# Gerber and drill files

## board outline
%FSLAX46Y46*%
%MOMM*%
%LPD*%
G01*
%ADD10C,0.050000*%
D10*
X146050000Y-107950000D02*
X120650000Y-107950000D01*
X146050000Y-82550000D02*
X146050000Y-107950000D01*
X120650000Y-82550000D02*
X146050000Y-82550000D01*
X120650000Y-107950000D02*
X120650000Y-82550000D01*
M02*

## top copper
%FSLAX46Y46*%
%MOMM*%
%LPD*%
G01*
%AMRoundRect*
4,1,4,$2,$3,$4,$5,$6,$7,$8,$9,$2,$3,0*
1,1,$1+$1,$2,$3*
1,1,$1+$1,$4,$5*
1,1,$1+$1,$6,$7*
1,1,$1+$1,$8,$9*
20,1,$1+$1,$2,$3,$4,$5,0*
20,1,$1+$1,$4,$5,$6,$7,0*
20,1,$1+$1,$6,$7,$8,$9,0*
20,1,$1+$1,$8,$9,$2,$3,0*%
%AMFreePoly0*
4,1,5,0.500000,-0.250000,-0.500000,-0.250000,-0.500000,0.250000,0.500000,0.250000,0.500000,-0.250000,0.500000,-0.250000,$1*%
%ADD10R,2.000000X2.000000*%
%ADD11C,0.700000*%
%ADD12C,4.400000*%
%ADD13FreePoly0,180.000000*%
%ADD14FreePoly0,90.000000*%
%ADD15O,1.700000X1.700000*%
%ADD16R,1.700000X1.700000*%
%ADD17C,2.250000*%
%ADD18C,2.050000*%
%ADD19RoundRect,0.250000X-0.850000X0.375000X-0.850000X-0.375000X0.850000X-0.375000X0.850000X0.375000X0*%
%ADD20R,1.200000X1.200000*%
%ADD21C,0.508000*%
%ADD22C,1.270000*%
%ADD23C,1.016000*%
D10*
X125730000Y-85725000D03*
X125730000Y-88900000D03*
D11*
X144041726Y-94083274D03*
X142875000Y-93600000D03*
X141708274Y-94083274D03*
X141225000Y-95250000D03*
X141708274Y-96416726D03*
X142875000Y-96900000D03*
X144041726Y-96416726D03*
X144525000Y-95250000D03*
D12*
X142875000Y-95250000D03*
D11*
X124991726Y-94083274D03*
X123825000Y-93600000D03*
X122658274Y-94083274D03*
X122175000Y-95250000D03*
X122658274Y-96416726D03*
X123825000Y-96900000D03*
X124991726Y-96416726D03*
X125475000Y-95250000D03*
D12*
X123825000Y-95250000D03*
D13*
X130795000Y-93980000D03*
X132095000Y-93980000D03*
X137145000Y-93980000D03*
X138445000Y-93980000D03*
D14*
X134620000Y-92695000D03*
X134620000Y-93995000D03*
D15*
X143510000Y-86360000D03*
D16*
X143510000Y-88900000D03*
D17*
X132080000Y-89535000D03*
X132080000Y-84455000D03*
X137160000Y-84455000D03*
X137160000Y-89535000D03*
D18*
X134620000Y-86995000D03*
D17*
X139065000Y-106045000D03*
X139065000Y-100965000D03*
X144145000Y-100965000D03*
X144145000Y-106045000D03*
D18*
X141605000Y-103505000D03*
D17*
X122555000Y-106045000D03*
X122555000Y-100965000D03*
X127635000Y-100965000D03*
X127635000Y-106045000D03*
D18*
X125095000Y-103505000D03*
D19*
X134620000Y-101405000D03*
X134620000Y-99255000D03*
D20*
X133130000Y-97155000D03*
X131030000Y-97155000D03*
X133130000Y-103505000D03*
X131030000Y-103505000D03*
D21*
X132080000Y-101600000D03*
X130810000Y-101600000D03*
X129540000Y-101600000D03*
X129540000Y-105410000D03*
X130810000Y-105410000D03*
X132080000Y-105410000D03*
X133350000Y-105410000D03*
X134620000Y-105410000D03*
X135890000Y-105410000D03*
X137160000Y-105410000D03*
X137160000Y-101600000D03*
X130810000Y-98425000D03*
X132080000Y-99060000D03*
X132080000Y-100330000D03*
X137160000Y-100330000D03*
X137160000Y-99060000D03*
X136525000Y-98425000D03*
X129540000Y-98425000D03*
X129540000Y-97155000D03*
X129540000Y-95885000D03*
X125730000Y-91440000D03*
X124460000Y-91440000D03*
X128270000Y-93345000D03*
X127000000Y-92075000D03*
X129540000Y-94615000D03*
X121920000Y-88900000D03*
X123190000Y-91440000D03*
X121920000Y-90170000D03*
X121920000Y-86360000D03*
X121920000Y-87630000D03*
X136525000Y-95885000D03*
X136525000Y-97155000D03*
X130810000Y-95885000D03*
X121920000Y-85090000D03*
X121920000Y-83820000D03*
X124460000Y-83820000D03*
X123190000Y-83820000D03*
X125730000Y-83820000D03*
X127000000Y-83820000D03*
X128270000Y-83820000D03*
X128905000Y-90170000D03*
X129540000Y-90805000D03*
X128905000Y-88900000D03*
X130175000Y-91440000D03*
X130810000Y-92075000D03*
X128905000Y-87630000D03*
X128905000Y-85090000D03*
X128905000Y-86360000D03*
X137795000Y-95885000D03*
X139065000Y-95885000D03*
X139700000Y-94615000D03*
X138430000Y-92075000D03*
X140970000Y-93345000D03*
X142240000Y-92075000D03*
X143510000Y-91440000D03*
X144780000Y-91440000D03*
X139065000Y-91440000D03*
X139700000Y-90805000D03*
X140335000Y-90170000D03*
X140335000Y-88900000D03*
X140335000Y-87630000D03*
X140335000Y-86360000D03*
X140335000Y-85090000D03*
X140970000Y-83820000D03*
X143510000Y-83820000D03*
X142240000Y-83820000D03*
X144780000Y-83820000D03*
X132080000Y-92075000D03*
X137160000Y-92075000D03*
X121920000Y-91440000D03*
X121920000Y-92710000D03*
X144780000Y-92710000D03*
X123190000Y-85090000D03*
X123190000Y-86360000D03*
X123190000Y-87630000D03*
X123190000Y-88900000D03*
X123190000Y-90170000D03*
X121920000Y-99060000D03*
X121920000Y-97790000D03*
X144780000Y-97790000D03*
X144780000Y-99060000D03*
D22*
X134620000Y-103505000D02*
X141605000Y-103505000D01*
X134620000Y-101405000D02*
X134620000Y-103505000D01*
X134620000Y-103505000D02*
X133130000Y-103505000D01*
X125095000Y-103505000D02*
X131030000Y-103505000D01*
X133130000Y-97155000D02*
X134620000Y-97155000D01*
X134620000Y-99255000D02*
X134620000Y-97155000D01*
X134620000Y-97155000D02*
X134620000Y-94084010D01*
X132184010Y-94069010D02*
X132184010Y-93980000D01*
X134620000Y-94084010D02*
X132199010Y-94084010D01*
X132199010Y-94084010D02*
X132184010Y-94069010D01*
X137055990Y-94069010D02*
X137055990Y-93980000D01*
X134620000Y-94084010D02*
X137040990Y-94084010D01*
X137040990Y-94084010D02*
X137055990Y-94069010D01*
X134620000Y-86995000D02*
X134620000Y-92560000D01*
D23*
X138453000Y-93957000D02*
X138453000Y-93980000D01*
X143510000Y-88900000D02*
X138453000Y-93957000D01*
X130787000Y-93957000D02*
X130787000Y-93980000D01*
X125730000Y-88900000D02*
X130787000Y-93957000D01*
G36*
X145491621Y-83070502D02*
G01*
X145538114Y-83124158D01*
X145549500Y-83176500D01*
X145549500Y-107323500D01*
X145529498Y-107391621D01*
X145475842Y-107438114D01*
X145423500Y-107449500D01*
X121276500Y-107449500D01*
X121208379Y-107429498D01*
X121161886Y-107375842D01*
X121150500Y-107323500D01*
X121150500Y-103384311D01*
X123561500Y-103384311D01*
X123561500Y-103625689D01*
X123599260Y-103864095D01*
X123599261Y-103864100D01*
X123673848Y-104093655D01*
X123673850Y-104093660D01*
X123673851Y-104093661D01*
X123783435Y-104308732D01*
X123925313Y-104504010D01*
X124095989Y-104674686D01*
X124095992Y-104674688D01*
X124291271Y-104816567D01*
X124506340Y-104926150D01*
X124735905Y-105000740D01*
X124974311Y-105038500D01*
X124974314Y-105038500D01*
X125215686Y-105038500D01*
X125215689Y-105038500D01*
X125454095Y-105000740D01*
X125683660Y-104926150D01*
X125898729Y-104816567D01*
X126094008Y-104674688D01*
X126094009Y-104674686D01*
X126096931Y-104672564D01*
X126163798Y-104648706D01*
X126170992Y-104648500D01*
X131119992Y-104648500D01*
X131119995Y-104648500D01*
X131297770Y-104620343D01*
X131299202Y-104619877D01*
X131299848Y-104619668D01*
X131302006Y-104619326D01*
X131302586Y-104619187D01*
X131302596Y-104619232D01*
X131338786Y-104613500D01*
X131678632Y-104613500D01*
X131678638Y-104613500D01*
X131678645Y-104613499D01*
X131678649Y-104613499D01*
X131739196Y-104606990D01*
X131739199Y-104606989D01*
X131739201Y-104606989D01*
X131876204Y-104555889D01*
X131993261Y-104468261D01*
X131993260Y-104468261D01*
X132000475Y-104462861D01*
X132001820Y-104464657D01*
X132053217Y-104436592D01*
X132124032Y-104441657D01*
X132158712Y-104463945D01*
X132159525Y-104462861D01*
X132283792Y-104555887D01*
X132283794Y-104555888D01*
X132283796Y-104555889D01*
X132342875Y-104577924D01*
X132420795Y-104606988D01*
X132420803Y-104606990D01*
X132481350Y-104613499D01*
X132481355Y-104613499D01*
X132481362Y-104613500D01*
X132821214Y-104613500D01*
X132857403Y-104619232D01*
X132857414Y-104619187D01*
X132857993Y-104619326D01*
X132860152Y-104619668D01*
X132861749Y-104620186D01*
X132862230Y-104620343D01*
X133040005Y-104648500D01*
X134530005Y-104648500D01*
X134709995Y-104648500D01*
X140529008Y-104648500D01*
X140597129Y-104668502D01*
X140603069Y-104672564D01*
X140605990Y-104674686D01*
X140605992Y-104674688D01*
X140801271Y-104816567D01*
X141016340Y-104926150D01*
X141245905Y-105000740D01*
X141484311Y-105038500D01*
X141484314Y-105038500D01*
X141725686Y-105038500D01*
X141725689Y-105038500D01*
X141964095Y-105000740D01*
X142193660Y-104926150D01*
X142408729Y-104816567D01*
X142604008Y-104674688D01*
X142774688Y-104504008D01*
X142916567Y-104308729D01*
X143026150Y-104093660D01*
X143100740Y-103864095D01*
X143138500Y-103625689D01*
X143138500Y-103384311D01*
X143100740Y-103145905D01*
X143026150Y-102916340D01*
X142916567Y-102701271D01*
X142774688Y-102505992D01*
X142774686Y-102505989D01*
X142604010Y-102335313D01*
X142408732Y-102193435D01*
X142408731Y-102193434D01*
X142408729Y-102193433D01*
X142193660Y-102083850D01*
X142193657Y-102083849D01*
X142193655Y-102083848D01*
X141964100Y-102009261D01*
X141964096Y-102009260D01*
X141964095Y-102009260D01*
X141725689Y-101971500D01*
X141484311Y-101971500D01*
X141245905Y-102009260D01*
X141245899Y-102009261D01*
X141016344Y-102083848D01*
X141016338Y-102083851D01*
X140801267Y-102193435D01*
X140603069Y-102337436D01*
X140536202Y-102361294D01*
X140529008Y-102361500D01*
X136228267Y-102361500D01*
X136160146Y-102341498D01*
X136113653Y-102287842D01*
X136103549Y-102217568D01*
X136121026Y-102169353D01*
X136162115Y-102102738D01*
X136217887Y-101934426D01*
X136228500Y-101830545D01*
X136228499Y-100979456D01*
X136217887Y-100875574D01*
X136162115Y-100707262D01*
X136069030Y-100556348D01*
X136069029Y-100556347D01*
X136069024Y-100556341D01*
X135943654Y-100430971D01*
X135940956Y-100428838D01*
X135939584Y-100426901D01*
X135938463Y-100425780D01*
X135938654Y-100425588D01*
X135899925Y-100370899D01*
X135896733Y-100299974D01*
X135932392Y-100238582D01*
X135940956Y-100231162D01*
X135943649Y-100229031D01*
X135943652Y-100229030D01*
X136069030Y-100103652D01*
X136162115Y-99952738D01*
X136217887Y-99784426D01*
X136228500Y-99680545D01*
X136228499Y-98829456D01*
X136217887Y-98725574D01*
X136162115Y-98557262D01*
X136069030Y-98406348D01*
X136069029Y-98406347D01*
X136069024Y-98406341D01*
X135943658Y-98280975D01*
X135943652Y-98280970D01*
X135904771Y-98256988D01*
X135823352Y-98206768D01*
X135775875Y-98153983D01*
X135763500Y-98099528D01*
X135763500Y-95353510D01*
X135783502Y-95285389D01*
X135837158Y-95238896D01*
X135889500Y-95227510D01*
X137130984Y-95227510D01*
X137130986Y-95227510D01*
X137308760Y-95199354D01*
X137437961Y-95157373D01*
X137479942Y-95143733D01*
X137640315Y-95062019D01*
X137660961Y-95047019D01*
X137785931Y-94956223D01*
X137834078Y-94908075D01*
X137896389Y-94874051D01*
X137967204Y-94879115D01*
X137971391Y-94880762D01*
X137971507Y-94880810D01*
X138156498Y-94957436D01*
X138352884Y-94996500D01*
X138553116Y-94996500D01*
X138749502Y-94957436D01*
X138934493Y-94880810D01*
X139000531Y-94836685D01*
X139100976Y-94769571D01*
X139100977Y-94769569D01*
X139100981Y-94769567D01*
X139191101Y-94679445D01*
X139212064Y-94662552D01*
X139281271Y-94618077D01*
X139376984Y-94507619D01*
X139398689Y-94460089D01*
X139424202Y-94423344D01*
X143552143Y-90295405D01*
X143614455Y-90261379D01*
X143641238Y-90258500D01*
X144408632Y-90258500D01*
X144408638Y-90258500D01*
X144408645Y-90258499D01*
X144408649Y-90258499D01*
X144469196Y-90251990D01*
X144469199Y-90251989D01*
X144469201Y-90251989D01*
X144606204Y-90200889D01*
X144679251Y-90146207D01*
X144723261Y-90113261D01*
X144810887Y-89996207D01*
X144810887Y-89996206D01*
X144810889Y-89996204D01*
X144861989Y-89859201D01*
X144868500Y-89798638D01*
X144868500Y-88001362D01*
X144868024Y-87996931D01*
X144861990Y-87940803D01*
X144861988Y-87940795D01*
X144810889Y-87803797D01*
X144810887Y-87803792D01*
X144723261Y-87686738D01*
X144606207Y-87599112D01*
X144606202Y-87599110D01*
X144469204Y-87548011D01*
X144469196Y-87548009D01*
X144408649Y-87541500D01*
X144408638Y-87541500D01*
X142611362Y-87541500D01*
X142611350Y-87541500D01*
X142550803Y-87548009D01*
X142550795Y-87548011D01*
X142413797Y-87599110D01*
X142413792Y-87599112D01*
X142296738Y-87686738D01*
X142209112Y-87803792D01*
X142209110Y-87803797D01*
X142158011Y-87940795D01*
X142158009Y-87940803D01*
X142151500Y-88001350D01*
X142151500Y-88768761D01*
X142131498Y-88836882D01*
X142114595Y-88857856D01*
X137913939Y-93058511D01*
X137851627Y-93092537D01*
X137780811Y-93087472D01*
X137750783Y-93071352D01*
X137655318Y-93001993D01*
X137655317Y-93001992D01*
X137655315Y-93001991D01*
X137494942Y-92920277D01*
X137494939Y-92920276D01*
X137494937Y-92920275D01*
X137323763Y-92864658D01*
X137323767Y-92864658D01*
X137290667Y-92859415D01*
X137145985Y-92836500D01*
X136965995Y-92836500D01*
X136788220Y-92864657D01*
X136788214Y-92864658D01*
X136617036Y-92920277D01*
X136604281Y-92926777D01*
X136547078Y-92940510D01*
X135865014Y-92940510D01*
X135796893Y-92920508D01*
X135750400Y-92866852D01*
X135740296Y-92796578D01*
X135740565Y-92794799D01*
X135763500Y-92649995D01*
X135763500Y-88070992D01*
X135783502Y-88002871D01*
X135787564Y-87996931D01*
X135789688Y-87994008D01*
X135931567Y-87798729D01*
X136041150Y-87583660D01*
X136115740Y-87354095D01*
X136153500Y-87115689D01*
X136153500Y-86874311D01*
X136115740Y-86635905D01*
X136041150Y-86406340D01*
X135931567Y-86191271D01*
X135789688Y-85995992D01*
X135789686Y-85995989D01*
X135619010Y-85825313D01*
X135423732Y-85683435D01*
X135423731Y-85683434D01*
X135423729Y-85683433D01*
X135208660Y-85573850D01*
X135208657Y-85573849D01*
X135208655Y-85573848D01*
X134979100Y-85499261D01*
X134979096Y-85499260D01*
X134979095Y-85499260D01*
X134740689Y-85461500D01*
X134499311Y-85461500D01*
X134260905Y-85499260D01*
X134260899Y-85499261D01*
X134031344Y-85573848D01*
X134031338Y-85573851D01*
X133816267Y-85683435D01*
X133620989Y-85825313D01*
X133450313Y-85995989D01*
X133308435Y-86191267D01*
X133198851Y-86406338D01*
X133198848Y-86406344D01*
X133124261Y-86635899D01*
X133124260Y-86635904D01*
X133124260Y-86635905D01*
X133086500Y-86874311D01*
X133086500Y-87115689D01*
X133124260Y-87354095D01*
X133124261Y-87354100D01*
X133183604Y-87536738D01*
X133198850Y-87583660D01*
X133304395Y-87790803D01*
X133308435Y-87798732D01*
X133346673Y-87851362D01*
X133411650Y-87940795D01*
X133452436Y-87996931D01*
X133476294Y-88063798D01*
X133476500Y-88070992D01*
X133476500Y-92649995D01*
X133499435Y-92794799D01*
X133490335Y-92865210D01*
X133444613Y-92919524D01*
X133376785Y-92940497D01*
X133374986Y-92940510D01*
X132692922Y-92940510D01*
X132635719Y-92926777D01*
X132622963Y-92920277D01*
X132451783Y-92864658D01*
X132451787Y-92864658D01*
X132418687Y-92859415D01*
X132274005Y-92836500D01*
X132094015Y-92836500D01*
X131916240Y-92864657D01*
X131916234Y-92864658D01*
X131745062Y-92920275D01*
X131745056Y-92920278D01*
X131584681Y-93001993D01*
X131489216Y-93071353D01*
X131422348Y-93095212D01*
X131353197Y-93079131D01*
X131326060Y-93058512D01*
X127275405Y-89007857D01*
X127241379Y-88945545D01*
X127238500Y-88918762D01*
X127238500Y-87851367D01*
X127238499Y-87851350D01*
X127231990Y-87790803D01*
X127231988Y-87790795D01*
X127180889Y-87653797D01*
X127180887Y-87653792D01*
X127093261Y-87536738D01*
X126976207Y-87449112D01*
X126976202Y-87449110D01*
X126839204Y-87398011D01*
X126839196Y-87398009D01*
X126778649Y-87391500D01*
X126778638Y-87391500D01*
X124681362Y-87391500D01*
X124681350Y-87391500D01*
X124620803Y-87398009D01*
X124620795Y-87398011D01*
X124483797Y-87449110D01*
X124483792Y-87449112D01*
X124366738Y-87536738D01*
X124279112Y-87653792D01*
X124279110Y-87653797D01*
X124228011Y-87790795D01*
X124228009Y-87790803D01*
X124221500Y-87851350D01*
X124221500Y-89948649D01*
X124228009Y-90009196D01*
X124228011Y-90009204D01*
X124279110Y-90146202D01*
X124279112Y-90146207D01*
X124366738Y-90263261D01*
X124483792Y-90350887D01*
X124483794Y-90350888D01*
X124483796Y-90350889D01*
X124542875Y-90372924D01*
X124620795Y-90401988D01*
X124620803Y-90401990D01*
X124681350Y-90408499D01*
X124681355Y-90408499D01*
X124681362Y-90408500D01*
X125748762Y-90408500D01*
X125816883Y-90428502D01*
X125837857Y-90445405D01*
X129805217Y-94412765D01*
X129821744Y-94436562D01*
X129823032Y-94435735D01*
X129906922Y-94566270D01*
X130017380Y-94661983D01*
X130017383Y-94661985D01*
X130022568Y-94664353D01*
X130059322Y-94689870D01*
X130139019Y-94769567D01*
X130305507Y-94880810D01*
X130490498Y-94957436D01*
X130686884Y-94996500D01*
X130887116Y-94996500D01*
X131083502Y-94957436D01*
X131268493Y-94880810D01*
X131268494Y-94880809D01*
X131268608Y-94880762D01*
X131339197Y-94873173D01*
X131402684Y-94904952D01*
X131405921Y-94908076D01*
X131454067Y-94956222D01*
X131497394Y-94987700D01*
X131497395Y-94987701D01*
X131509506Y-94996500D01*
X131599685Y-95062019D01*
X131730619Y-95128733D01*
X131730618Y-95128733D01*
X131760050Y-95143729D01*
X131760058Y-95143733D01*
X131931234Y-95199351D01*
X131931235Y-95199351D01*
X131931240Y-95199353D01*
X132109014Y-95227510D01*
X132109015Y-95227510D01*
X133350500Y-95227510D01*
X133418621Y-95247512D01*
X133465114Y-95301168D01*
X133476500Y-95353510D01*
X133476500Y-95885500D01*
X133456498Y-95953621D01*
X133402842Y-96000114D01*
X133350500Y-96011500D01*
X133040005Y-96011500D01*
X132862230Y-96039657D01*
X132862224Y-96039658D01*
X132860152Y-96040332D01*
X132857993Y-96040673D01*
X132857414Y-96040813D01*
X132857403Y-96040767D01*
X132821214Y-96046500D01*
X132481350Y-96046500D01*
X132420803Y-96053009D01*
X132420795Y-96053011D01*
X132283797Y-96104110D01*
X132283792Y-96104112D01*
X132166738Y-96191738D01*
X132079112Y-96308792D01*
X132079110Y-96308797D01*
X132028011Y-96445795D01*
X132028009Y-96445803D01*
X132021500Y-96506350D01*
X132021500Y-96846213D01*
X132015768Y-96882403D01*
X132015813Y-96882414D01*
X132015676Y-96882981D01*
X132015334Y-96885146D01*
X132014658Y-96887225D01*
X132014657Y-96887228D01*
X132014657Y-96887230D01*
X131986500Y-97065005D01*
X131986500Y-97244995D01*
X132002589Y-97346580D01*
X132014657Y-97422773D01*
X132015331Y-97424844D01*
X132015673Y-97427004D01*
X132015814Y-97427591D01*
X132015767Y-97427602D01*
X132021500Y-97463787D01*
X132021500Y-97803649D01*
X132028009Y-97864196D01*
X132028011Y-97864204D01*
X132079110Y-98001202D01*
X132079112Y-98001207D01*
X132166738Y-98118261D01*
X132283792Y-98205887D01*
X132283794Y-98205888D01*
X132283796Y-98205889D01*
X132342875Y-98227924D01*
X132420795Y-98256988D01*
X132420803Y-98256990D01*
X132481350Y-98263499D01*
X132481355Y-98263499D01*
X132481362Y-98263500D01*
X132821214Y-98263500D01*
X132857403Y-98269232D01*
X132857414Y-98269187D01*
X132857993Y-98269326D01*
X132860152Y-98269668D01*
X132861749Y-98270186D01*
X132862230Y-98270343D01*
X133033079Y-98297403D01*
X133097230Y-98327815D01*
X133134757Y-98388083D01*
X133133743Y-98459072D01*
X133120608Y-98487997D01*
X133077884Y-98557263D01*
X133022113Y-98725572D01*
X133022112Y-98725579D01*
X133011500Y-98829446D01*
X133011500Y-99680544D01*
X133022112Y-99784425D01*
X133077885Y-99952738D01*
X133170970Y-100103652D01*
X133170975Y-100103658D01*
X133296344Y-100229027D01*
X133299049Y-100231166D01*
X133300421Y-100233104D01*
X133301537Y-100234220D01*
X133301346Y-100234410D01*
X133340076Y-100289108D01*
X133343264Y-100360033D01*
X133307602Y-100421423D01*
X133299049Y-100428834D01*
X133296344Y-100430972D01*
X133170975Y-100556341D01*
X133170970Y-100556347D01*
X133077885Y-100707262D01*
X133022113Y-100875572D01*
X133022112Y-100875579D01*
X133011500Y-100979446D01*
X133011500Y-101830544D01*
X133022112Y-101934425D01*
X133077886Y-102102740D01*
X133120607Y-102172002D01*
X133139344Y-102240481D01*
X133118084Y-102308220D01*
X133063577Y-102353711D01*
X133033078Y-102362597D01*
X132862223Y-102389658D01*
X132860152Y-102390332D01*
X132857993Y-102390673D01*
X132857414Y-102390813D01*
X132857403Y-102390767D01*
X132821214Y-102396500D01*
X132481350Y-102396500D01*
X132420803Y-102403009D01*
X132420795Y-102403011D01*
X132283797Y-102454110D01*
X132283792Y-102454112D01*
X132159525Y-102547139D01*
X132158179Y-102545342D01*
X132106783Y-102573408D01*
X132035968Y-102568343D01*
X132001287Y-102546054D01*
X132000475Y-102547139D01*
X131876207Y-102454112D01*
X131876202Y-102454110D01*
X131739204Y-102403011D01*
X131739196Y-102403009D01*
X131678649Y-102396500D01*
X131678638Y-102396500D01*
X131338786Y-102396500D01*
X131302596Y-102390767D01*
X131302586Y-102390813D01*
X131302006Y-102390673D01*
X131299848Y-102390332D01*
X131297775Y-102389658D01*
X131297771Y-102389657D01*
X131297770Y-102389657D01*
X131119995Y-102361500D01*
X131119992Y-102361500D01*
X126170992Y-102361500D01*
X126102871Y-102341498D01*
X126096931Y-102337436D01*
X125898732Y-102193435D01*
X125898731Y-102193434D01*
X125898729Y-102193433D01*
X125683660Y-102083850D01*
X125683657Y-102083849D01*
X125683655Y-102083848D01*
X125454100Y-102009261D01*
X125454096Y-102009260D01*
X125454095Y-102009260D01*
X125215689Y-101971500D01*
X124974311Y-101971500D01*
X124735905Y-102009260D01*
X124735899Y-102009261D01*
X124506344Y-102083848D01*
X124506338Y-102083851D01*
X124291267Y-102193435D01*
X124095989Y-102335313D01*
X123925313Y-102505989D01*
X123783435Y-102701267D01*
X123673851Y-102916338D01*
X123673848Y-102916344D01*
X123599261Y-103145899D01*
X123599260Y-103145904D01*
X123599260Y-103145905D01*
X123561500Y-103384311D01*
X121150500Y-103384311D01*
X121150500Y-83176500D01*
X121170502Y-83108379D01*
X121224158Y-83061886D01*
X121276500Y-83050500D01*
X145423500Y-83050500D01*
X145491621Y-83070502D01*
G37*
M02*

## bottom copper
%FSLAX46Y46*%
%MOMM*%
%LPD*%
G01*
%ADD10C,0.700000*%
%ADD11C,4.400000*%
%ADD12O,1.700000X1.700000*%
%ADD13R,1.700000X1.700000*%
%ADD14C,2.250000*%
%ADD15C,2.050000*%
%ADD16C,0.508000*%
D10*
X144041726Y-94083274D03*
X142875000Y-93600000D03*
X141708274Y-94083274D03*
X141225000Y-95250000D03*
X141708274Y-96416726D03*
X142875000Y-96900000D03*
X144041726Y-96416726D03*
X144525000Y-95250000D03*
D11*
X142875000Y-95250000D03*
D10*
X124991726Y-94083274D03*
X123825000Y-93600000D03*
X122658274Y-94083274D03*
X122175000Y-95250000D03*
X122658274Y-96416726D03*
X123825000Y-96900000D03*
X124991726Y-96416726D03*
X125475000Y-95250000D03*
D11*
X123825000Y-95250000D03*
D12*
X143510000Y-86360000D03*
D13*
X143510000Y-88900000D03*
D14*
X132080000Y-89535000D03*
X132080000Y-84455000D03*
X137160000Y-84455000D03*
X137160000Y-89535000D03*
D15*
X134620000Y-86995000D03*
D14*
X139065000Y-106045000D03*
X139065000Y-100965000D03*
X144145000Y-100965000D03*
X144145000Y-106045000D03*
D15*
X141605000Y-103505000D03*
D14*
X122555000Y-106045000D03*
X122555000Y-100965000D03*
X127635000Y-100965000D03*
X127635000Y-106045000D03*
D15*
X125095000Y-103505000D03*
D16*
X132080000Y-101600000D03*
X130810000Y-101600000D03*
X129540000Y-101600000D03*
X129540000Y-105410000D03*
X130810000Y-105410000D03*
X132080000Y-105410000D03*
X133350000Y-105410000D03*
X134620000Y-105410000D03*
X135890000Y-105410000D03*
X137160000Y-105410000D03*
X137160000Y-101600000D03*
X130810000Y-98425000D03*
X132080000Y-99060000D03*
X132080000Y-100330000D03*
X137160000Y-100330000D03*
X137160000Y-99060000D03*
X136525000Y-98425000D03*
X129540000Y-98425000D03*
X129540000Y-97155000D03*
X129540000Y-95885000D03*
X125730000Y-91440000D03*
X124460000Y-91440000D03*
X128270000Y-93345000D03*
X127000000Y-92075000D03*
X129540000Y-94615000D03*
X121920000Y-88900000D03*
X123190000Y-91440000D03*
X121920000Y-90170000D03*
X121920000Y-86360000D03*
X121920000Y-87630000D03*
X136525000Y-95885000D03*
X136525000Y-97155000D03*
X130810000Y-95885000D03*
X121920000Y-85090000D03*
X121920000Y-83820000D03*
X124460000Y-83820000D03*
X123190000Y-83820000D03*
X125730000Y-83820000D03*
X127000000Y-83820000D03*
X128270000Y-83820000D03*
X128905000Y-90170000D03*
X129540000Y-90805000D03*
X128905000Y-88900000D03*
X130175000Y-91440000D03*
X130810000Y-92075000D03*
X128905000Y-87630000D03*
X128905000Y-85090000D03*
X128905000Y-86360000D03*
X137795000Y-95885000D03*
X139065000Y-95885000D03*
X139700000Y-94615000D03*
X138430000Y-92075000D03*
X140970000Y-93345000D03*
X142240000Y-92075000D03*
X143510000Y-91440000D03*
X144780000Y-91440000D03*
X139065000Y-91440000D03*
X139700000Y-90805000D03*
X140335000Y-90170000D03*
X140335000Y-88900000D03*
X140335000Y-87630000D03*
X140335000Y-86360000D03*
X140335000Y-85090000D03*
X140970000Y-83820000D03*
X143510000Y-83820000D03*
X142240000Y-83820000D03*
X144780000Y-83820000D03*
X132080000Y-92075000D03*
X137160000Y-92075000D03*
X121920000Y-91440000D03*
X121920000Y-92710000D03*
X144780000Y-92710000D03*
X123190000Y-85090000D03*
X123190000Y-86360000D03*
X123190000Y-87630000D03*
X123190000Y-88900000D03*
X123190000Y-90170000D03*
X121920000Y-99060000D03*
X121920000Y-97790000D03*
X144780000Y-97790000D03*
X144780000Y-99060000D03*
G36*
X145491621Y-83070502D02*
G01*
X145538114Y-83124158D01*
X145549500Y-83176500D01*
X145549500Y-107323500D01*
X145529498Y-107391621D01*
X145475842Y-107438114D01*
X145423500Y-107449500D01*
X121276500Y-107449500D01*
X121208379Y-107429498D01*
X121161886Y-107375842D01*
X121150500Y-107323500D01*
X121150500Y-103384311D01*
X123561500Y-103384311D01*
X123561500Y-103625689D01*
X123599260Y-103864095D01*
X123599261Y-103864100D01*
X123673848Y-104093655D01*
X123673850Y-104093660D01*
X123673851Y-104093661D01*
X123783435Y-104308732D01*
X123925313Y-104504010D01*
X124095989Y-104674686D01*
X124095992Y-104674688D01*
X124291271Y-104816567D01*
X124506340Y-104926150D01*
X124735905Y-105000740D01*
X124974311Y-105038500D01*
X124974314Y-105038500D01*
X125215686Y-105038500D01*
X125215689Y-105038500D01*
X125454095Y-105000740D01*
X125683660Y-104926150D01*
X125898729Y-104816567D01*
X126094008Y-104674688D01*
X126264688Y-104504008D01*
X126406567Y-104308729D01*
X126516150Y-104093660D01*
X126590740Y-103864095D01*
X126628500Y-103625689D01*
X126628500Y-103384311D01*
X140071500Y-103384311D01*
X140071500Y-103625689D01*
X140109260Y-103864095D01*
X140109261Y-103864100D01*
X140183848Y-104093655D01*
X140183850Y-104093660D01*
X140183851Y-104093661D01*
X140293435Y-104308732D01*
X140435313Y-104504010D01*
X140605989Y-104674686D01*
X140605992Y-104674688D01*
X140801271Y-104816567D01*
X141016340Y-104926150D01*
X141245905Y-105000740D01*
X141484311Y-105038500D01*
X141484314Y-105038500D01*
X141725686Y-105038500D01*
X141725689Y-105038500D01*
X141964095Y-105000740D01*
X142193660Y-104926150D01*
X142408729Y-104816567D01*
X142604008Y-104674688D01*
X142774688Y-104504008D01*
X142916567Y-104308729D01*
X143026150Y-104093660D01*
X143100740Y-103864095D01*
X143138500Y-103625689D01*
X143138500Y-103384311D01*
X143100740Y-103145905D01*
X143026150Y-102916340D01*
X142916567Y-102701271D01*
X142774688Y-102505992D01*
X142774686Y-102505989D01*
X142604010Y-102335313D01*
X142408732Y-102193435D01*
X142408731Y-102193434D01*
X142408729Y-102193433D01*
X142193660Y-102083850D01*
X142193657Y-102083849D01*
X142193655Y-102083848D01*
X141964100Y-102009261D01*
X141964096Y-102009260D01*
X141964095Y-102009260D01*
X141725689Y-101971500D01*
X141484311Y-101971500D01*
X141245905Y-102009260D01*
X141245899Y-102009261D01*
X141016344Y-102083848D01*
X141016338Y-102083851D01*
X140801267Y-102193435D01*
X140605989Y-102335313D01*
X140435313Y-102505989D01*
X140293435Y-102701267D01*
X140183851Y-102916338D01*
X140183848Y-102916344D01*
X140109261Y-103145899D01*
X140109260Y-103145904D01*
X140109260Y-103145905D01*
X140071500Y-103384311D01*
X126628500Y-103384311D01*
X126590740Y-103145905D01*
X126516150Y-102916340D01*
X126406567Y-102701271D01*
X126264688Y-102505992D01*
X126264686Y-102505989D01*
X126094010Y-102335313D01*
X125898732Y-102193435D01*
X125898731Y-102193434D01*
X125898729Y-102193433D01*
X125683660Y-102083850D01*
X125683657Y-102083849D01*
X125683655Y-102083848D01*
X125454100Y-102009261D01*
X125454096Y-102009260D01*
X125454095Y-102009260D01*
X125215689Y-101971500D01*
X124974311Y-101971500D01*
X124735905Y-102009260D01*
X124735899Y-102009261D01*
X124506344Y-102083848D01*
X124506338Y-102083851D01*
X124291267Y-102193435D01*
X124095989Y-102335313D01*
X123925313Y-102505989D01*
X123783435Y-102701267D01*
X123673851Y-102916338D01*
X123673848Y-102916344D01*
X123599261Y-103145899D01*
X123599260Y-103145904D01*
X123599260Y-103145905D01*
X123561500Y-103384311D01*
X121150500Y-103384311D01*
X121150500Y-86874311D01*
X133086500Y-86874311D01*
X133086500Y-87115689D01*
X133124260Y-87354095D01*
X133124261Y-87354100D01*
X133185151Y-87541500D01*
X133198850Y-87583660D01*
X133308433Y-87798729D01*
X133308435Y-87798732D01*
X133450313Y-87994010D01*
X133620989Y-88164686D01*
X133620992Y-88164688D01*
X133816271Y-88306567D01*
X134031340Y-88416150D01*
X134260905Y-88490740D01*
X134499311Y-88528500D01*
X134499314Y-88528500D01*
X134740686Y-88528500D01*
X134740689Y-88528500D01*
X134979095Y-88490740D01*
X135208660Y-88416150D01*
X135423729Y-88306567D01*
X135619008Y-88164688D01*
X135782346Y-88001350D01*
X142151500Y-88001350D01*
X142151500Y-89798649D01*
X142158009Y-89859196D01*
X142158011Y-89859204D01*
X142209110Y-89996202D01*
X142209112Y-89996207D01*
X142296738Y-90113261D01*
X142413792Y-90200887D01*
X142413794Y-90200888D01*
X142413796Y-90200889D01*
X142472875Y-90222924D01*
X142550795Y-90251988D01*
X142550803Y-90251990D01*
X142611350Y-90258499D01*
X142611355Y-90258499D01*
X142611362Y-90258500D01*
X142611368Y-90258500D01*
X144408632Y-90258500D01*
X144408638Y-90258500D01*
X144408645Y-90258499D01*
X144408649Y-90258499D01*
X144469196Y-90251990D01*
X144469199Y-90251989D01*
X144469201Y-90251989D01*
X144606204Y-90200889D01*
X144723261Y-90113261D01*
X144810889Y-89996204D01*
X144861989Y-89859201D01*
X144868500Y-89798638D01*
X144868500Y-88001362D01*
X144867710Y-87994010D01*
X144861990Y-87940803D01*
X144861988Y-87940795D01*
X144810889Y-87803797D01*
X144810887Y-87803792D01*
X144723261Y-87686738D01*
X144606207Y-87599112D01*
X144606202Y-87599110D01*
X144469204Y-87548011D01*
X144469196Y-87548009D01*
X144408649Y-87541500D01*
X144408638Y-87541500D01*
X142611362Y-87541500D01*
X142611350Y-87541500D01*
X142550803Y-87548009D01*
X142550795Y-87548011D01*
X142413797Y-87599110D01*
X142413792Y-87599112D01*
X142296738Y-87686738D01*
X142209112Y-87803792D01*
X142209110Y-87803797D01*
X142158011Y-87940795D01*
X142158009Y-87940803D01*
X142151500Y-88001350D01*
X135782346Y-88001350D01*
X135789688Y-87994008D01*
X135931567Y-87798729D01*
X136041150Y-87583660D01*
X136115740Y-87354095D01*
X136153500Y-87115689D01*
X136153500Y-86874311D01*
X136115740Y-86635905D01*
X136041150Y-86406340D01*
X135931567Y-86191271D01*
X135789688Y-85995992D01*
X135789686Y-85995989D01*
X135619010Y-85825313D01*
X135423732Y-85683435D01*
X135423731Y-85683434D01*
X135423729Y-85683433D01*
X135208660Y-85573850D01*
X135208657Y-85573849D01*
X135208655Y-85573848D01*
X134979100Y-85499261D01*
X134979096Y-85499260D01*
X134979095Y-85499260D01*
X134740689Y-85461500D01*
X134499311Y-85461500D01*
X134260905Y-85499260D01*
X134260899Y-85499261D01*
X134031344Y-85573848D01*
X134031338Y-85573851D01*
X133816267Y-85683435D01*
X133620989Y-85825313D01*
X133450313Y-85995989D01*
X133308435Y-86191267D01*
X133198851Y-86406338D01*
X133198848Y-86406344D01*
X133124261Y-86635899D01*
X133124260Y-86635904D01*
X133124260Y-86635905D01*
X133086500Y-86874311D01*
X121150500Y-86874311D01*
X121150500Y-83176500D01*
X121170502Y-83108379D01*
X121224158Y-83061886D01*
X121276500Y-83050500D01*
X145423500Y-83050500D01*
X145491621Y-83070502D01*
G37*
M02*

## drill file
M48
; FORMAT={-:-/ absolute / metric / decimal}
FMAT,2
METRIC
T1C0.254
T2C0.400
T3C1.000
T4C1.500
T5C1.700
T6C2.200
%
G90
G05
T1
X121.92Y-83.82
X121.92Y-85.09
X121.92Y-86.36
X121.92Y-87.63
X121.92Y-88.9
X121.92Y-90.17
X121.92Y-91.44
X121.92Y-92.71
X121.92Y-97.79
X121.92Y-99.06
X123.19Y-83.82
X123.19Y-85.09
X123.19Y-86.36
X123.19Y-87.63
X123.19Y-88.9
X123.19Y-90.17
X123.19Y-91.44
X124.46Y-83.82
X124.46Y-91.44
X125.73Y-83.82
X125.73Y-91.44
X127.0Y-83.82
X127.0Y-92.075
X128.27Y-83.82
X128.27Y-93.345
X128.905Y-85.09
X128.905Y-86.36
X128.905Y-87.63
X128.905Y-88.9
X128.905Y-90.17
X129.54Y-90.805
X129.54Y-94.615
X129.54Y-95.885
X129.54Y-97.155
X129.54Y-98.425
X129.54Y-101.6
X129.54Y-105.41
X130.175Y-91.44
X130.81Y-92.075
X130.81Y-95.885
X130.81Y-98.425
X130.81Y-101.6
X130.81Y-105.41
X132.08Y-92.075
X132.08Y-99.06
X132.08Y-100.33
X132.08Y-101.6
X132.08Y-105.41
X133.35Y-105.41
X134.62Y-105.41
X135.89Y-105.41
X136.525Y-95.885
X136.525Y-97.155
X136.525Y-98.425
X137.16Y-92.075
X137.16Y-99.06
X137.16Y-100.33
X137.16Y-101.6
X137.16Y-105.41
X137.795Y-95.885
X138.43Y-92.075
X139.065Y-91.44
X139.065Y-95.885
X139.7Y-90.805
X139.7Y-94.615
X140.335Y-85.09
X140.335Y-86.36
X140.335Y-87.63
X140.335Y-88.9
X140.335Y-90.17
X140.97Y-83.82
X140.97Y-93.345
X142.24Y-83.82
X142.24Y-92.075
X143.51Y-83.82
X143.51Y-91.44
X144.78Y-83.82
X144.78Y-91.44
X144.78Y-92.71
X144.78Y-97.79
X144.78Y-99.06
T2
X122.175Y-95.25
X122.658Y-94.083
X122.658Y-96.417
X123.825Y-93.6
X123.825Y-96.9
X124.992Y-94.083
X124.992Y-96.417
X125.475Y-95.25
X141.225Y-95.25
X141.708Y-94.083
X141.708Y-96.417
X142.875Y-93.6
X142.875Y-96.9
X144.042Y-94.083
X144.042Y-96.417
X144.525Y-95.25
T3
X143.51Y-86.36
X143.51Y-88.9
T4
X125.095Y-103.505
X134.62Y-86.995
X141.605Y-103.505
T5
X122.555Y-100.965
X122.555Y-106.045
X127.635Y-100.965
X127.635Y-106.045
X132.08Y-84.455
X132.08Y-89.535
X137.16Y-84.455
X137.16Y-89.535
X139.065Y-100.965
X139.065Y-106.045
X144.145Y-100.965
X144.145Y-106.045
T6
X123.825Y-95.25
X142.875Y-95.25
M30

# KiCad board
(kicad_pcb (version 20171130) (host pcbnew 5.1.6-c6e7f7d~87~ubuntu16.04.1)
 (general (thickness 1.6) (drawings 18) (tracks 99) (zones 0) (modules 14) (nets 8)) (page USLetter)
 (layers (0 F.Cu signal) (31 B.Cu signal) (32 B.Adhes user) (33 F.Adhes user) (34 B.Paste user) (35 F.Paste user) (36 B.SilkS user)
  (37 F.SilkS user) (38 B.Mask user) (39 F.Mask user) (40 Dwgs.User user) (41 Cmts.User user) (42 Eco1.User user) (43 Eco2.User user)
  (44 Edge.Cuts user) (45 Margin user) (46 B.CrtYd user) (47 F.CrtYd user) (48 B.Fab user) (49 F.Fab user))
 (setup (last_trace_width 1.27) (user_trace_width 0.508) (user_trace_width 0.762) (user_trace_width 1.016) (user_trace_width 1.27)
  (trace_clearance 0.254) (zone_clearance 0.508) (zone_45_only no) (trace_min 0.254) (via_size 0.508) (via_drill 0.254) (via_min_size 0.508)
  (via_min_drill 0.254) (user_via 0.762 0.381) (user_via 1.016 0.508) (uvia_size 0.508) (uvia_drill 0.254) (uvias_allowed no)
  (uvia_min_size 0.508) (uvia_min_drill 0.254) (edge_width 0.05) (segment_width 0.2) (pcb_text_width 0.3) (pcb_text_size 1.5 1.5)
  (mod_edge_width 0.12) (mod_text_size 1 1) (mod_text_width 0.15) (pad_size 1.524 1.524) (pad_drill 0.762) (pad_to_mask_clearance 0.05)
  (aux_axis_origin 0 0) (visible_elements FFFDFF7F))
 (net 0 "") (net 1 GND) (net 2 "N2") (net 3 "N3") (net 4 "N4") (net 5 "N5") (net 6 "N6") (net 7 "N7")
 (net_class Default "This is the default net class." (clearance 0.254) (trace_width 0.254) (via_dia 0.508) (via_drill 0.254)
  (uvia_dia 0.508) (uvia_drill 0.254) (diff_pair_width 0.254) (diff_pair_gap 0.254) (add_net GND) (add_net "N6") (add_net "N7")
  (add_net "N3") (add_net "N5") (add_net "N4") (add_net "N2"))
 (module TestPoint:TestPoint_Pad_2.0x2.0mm (layer F.Cu) (at 125.73 85.725)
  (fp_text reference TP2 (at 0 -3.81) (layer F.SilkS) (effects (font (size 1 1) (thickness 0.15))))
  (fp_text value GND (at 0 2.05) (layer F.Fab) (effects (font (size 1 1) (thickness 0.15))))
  (pad 1 smd rect (at 0 0) (size 2 2) (layers F.Cu F.Mask) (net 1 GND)))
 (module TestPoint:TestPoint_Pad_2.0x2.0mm (layer F.Cu) (at 125.73 88.9)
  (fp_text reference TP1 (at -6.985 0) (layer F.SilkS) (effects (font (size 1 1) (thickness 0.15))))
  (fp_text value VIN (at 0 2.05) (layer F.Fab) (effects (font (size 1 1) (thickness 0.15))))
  (pad 1 smd rect (at 0 0) (size 2 2) (layers F.Cu F.Mask) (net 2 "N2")))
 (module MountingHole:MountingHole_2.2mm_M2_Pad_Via (layer F.Cu) (at 142.875 95.25)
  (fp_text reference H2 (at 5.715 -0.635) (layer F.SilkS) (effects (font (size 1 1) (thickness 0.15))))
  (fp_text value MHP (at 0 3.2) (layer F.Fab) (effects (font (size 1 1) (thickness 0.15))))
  (pad 1 thru_hole circle (at 1.166726 -1.166726) (size 0.7 0.7) (drill 0.4) (layers *.Cu *.Mask) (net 1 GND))
  (pad 1 thru_hole circle (at 0 -1.65) (size 0.7 0.7) (drill 0.4) (layers *.Cu *.Mask) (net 1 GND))
  (pad 1 thru_hole circle (at -1.166726 -1.166726) (size 0.7 0.7) (drill 0.4) (layers *.Cu *.Mask) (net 1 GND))
  (pad 1 thru_hole circle (at -1.65 0) (size 0.7 0.7) (drill 0.4) (layers *.Cu *.Mask) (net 1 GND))
  (pad 1 thru_hole circle (at -1.166726 1.166726) (size 0.7 0.7) (drill 0.4) (layers *.Cu *.Mask) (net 1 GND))
  (pad 1 thru_hole circle (at 0 1.65) (size 0.7 0.7) (drill 0.4) (layers *.Cu *.Mask) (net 1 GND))
  (pad 1 thru_hole circle (at 1.166726 1.166726) (size 0.7 0.7) (drill 0.4) (layers *.Cu *.Mask) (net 1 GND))
  (pad 1 thru_hole circle (at 1.65 0) (size 0.7 0.7) (drill 0.4) (layers *.Cu *.Mask) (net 1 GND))
  (pad 1 thru_hole circle (at 0 0) (size 4.4 4.4) (drill 2.2) (layers *.Cu *.Mask) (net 1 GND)))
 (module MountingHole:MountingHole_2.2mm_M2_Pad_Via (layer F.Cu) (at 123.825 95.25)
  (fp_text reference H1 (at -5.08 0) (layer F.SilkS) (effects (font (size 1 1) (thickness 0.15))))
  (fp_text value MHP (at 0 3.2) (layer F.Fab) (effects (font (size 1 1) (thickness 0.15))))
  (pad 1 thru_hole circle (at 1.166726 -1.166726) (size 0.7 0.7) (drill 0.4) (layers *.Cu *.Mask) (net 1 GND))
  (pad 1 thru_hole circle (at 0 -1.65) (size 0.7 0.7) (drill 0.4) (layers *.Cu *.Mask) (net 1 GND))
  (pad 1 thru_hole circle (at -1.166726 -1.166726) (size 0.7 0.7) (drill 0.4) (layers *.Cu *.Mask) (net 1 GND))
  (pad 1 thru_hole circle (at -1.65 0) (size 0.7 0.7) (drill 0.4) (layers *.Cu *.Mask) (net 1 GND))
  (pad 1 thru_hole circle (at -1.166726 1.166726) (size 0.7 0.7) (drill 0.4) (layers *.Cu *.Mask) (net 1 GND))
  (pad 1 thru_hole circle (at 0 1.65) (size 0.7 0.7) (drill 0.4) (layers *.Cu *.Mask) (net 1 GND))
  (pad 1 thru_hole circle (at 1.166726 1.166726) (size 0.7 0.7) (drill 0.4) (layers *.Cu *.Mask) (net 1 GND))
  (pad 1 thru_hole circle (at 1.65 0) (size 0.7 0.7) (drill 0.4) (layers *.Cu *.Mask) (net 1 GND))
  (pad 1 thru_hole circle (at 0 0) (size 4.4 4.4) (drill 2.2) (layers *.Cu *.Mask) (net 1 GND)))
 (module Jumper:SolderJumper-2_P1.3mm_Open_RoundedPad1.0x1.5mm (layer F.Cu) (at 131.445 93.98 180)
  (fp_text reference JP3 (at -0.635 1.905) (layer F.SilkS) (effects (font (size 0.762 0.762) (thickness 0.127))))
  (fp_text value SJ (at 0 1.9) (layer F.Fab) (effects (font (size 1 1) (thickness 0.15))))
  (pad 2 smd custom (at 0.65 0 180) (size 1 0.5) (layers F.Cu F.Mask) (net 2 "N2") (zone_connect 2)
   (options (clearance outline) (anchor rect)) (primitives))
  (pad 1 smd custom (at -0.65 0 180) (size 1 0.5) (layers F.Cu F.Mask) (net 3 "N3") (zone_connect 2)
   (options (clearance outline) (anchor rect)) (primitives)))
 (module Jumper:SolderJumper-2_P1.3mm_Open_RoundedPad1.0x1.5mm (layer F.Cu) (at 137.795 93.98 180)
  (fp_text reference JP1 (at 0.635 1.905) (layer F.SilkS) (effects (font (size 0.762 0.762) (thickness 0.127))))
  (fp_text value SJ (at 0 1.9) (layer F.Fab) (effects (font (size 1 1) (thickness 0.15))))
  (pad 2 smd custom (at 0.65 0 180) (size 1 0.5) (layers F.Cu F.Mask) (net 3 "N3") (zone_connect 2)
   (options (clearance outline) (anchor rect)) (primitives))
  (pad 1 smd custom (at -0.65 0 180) (size 1 0.5) (layers F.Cu F.Mask) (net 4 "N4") (zone_connect 2)
   (options (clearance outline) (anchor rect)) (primitives)))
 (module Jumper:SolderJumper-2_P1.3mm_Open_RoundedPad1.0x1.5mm (layer F.Cu) (at 134.62 93.345 90)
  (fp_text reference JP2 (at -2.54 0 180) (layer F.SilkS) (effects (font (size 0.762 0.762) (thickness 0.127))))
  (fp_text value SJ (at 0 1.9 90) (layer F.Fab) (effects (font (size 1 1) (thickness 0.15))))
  (pad 2 smd custom (at 0.65 0 90) (size 1 0.5) (layers F.Cu F.Mask) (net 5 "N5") (zone_connect 2)
   (options (clearance outline) (anchor rect)) (primitives))
  (pad 1 smd custom (at -0.65 0 90) (size 1 0.5) (layers F.Cu F.Mask) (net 3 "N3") (zone_connect 2)
   (options (clearance outline) (anchor rect)) (primitives)))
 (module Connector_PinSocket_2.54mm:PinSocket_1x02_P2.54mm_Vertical (layer F.Cu) (at 143.51 88.9 180)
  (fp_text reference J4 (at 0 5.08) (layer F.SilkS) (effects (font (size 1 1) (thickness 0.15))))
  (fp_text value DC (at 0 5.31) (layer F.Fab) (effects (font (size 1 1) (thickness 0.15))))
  (pad 2 thru_hole oval (at 0 2.54 180) (size 1.7 1.7) (drill 1) (layers *.Cu *.Mask) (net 1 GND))
  (pad 1 thru_hole rect (at 0 0 180) (size 1.7 1.7) (drill 1) (layers *.Cu *.Mask) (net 4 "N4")))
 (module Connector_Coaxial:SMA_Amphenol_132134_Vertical (layer F.Cu) (at 134.62 86.995)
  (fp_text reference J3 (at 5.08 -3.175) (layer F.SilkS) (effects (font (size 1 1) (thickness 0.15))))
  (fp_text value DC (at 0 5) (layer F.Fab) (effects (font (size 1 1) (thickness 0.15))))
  (pad 2 thru_hole circle (at -2.54 2.54) (size 2.25 2.25) (drill 1.7) (layers *.Cu *.Mask) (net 1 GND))
  (pad 2 thru_hole circle (at -2.54 -2.54) (size 2.25 2.25) (drill 1.7) (layers *.Cu *.Mask) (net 1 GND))
  (pad 2 thru_hole circle (at 2.54 -2.54) (size 2.25 2.25) (drill 1.7) (layers *.Cu *.Mask) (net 1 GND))
  (pad 2 thru_hole circle (at 2.54 2.54) (size 2.25 2.25) (drill 1.7) (layers *.Cu *.Mask) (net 1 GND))
  (pad 1 thru_hole circle (at 0 0) (size 2.05 2.05) (drill 1.5) (layers *.Cu *.Mask) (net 5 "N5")))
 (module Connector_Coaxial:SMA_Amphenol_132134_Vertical (layer F.Cu) (at 141.605 103.505)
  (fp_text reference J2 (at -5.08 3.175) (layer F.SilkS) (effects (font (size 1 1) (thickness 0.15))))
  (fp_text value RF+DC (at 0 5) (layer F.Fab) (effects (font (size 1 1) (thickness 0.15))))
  (pad 2 thru_hole circle (at -2.54 2.54) (size 2.25 2.25) (drill 1.7) (layers *.Cu *.Mask) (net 1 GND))
  (pad 2 thru_hole circle (at -2.54 -2.54) (size 2.25 2.25) (drill 1.7) (layers *.Cu *.Mask) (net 1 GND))
  (pad 2 thru_hole circle (at 2.54 -2.54) (size 2.25 2.25) (drill 1.7) (layers *.Cu *.Mask) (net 1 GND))
  (pad 2 thru_hole circle (at 2.54 2.54) (size 2.25 2.25) (drill 1.7) (layers *.Cu *.Mask) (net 1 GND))
  (pad 1 thru_hole circle (at 0 0) (size 2.05 2.05) (drill 1.5) (layers *.Cu *.Mask) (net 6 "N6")))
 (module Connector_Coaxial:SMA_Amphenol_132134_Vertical (layer F.Cu) (at 125.095 103.505)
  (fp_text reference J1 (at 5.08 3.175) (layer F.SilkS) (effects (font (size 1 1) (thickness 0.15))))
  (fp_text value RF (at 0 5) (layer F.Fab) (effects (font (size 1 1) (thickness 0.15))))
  (pad 2 thru_hole circle (at -2.54 2.54) (size 2.25 2.25) (drill 1.7) (layers *.Cu *.Mask) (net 1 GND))
  (pad 2 thru_hole circle (at -2.54 -2.54) (size 2.25 2.25) (drill 1.7) (layers *.Cu *.Mask) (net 1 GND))
  (pad 2 thru_hole circle (at 2.54 -2.54) (size 2.25 2.25) (drill 1.7) (layers *.Cu *.Mask) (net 1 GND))
  (pad 2 thru_hole circle (at 2.54 2.54) (size 2.25 2.25) (drill 1.7) (layers *.Cu *.Mask) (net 1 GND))
  (pad 1 thru_hole circle (at 0 0) (size 2.05 2.05) (drill 1.5) (layers *.Cu *.Mask) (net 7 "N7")))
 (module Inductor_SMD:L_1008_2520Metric (layer F.Cu) (at 134.62 100.33 270)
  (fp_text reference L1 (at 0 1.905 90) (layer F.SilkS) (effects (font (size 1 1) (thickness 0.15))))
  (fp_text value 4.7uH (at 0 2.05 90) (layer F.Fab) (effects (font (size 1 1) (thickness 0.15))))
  (pad 2 smd roundrect (at 1.075 0 270) (size 1.25 2.2) (layers F.Cu F.Paste F.Mask) (roundrect_rratio 0.2) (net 6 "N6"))
  (pad 1 smd roundrect (at -1.075 0 270) (size 1.25 2.2) (layers F.Cu F.Paste F.Mask) (roundrect_rratio 0.2) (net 3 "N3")))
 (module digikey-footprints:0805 (layer F.Cu) (at 132.08 97.155 180)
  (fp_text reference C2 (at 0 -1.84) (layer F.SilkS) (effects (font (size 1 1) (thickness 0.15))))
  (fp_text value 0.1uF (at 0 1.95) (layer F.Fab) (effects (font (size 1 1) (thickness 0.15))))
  (pad 1 smd rect (at -1.05 0 180) (size 1.2 1.2) (layers F.Cu F.Paste F.Mask) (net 3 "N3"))
  (pad 2 smd rect (at 1.05 0 180) (size 1.2 1.2) (layers F.Cu F.Paste F.Mask) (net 1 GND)))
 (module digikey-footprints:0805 (layer F.Cu) (at 132.08 103.505 180)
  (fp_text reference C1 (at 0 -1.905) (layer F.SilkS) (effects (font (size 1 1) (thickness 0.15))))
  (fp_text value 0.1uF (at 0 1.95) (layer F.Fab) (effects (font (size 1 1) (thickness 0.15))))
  (pad 1 smd rect (at -1.05 0 180) (size 1.2 1.2) (layers F.Cu F.Paste F.Mask) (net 6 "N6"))
  (pad 2 smd rect (at 1.05 0 180) (size 1.2 1.2) (layers F.Cu F.Paste F.Mask) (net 7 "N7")))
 (gr_line (start 146.05 107.95) (end 120.65 107.95) (layer Edge.Cuts) (width 0.05))
 (gr_line (start 146.05 82.55) (end 146.05 107.95) (layer Edge.Cuts) (width 0.05))
 (gr_line (start 120.65 82.55) (end 146.05 82.55) (layer Edge.Cuts) (width 0.05))
 (gr_line (start 120.65 107.95) (end 120.65 82.55) (layer Edge.Cuts) (width 0.05))
 (segment (start 134.62 103.505) (end 141.605 103.505) (width 1.27) (layer F.Cu) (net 6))
 (segment (start 134.62 101.405) (end 134.62 103.505) (width 1.27) (layer F.Cu) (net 6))
 (segment (start 134.62 103.505) (end 133.13 103.505) (width 1.27) (layer F.Cu) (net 6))
 (segment (start 125.095 103.505) (end 131.03 103.505) (width 1.27) (layer F.Cu) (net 7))
 (segment (start 133.13 97.155) (end 134.62 97.155) (width 1.27) (layer F.Cu) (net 3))
 (segment (start 134.62 99.255) (end 134.62 97.155) (width 1.27) (layer F.Cu) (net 3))
 (segment (start 134.62 97.155) (end 134.62 94.08401) (width 1.27) (layer F.Cu) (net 3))
 (segment (start 132.18401 94.06901) (end 132.18401 93.98) (width 1.27) (layer F.Cu) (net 3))
 (segment (start 134.62 94.08401) (end 132.19901 94.08401) (width 1.27) (layer F.Cu) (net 3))
 (segment (start 132.19901 94.08401) (end 132.18401 94.06901) (width 1.27) (layer F.Cu) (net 3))
 (segment (start 137.05599 94.06901) (end 137.05599 93.98) (width 1.27) (layer F.Cu) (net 3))
 (segment (start 134.62 94.08401) (end 137.04099 94.08401) (width 1.27) (layer F.Cu) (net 3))
 (segment (start 137.04099 94.08401) (end 137.05599 94.06901) (width 1.27) (layer F.Cu) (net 3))
 (via (at 132.08 101.6) (size 0.508) (drill 0.254) (layers F.Cu B.Cu) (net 1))
 (via (at 130.81 101.6) (size 0.508) (drill 0.254) (layers F.Cu B.Cu) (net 1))
 (via (at 129.54 101.6) (size 0.508) (drill 0.254) (layers F.Cu B.Cu) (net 1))
 (via (at 129.54 105.41) (size 0.508) (drill 0.254) (layers F.Cu B.Cu) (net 1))
 (via (at 130.81 105.41) (size 0.508) (drill 0.254) (layers F.Cu B.Cu) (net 1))
 (via (at 132.08 105.41) (size 0.508) (drill 0.254) (layers F.Cu B.Cu) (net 1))
 (via (at 133.35 105.41) (size 0.508) (drill 0.254) (layers F.Cu B.Cu) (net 1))
 (via (at 134.62 105.41) (size 0.508) (drill 0.254) (layers F.Cu B.Cu) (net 1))
 (via (at 135.89 105.41) (size 0.508) (drill 0.254) (layers F.Cu B.Cu) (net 1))
 (via (at 137.16 105.41) (size 0.508) (drill 0.254) (layers F.Cu B.Cu) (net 1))
 (via (at 137.16 101.6) (size 0.508) (drill 0.254) (layers F.Cu B.Cu) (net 1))
 (via (at 130.81 98.425) (size 0.508) (drill 0.254) (layers F.Cu B.Cu) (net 1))
 (via (at 132.08 99.06) (size 0.508) (drill 0.254) (layers F.Cu B.Cu) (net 1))
 (via (at 132.08 100.33) (size 0.508) (drill 0.254) (layers F.Cu B.Cu) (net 1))
 (via (at 137.16 100.33) (size 0.508) (drill 0.254) (layers F.Cu B.Cu) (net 1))
 (via (at 137.16 99.06) (size 0.508) (drill 0.254) (layers F.Cu B.Cu) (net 1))
 (via (at 136.525 98.425) (size 0.508) (drill 0.254) (layers F.Cu B.Cu) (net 1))
 (via (at 129.54 98.425) (size 0.508) (drill 0.254) (layers F.Cu B.Cu) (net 1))
 (via (at 129.54 97.155) (size 0.508) (drill 0.254) (layers F.Cu B.Cu) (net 1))
 (via (at 129.54 95.885) (size 0.508) (drill 0.254) (layers F.Cu B.Cu) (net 1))
 (via (at 125.73 91.44) (size 0.508) (drill 0.254) (layers F.Cu B.Cu) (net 1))
 (via (at 124.46 91.44) (size 0.508) (drill 0.254) (layers F.Cu B.Cu) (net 1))
 (via (at 128.27 93.345) (size 0.508) (drill 0.254) (layers F.Cu B.Cu) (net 1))
 (via (at 127 92.075) (size 0.508) (drill 0.254) (layers F.Cu B.Cu) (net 1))
 (via (at 129.54 94.615) (size 0.508) (drill 0.254) (layers F.Cu B.Cu) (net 1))
 (via (at 121.92 88.9) (size 0.508) (drill 0.254) (layers F.Cu B.Cu) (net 1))
 (via (at 123.19 91.44) (size 0.508) (drill 0.254) (layers F.Cu B.Cu) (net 1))
 (via (at 121.92 90.17) (size 0.508) (drill 0.254) (layers F.Cu B.Cu) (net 1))
 (via (at 121.92 86.36) (size 0.508) (drill 0.254) (layers F.Cu B.Cu) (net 1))
 (via (at 121.92 87.63) (size 0.508) (drill 0.254) (layers F.Cu B.Cu) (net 1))
 (via (at 136.525 95.885) (size 0.508) (drill 0.254) (layers F.Cu B.Cu) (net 1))
 (via (at 136.525 97.155) (size 0.508) (drill 0.254) (layers F.Cu B.Cu) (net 1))
 (via (at 130.81 95.885) (size 0.508) (drill 0.254) (layers F.Cu B.Cu) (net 1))
 (via (at 121.92 85.09) (size 0.508) (drill 0.254) (layers F.Cu B.Cu) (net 1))
 (via (at 121.92 83.82) (size 0.508) (drill 0.254) (layers F.Cu B.Cu) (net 1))
 (via (at 124.46 83.82) (size 0.508) (drill 0.254) (layers F.Cu B.Cu) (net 1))
 (via (at 123.19 83.82) (size 0.508) (drill 0.254) (layers F.Cu B.Cu) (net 1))
 (via (at 125.73 83.82) (size 0.508) (drill 0.254) (layers F.Cu B.Cu) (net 1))
 (via (at 127 83.82) (size 0.508) (drill 0.254) (layers F.Cu B.Cu) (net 1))
 (via (at 128.27 83.82) (size 0.508) (drill 0.254) (layers F.Cu B.Cu) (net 1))
 (via (at 128.905 90.17) (size 0.508) (drill 0.254) (layers F.Cu B.Cu) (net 1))
 (via (at 129.54 90.805) (size 0.508) (drill 0.254) (layers F.Cu B.Cu) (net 1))
 (via (at 128.905 88.9) (size 0.508) (drill 0.254) (layers F.Cu B.Cu) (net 1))
 (via (at 130.175 91.44) (size 0.508) (drill 0.254) (layers F.Cu B.Cu) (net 1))
 (via (at 130.81 92.075) (size 0.508) (drill 0.254) (layers F.Cu B.Cu) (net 1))
 (via (at 128.905 87.63) (size 0.508) (drill 0.254) (layers F.Cu B.Cu) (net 1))
 (via (at 128.905 85.09) (size 0.508) (drill 0.254) (layers F.Cu B.Cu) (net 1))
 (via (at 128.905 86.36) (size 0.508) (drill 0.254) (layers F.Cu B.Cu) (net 1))
 (via (at 137.795 95.885) (size 0.508) (drill 0.254) (layers F.Cu B.Cu) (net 1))
 (via (at 139.065 95.885) (size 0.508) (drill 0.254) (layers F.Cu B.Cu) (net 1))
 (via (at 139.7 94.615) (size 0.508) (drill 0.254) (layers F.Cu B.Cu) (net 1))
 (via (at 138.43 92.075) (size 0.508) (drill 0.254) (layers F.Cu B.Cu) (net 1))
 (via (at 140.97 93.345) (size 0.508) (drill 0.254) (layers F.Cu B.Cu) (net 1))
 (via (at 142.24 92.075) (size 0.508) (drill 0.254) (layers F.Cu B.Cu) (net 1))
 (via (at 143.51 91.44) (size 0.508) (drill 0.254) (layers F.Cu B.Cu) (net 1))
 (via (at 144.78 91.44) (size 0.508) (drill 0.254) (layers F.Cu B.Cu) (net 1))
 (via (at 139.065 91.44) (size 0.508) (drill 0.254) (layers F.Cu B.Cu) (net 1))
 (via (at 139.7 90.805) (size 0.508) (drill 0.254) (layers F.Cu B.Cu) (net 1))
 (via (at 140.335 90.17) (size 0.508) (drill 0.254) (layers F.Cu B.Cu) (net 1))
 (via (at 140.335 88.9) (size 0.508) (drill 0.254) (layers F.Cu B.Cu) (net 1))
 (via (at 140.335 87.63) (size 0.508) (drill 0.254) (layers F.Cu B.Cu) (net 1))
 (via (at 140.335 86.36) (size 0.508) (drill 0.254) (layers F.Cu B.Cu) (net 1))
 (via (at 140.335 85.09) (size 0.508) (drill 0.254) (layers F.Cu B.Cu) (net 1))
 (via (at 140.97 83.82) (size 0.508) (drill 0.254) (layers F.Cu B.Cu) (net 1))
 (via (at 143.51 83.82) (size 0.508) (drill 0.254) (layers F.Cu B.Cu) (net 1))
 (via (at 142.24 83.82) (size 0.508) (drill 0.254) (layers F.Cu B.Cu) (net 1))
 (via (at 144.78 83.82) (size 0.508) (drill 0.254) (layers F.Cu B.Cu) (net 1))
 (via (at 132.08 92.075) (size 0.508) (drill 0.254) (layers F.Cu B.Cu) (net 1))
 (via (at 137.16 92.075) (size 0.508) (drill 0.254) (layers F.Cu B.Cu) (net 1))
 (via (at 121.92 91.44) (size 0.508) (drill 0.254) (layers F.Cu B.Cu) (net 1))
 (via (at 121.92 92.71) (size 0.508) (drill 0.254) (layers F.Cu B.Cu) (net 1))
 (via (at 144.78 92.71) (size 0.508) (drill 0.254) (layers F.Cu B.Cu) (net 1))
 (via (at 123.19 85.09) (size 0.508) (drill 0.254) (layers F.Cu B.Cu) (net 1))
 (via (at 123.19 86.36) (size 0.508) (drill 0.254) (layers F.Cu B.Cu) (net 1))
 (via (at 123.19 87.63) (size 0.508) (drill 0.254) (layers F.Cu B.Cu) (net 1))
 (via (at 123.19 88.9) (size 0.508) (drill 0.254) (layers F.Cu B.Cu) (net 1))
 (via (at 123.19 90.17) (size 0.508) (drill 0.254) (layers F.Cu B.Cu) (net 1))
 (via (at 121.92 99.06) (size 0.508) (drill 0.254) (layers F.Cu B.Cu) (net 1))
 (via (at 121.92 97.79) (size 0.508) (drill 0.254) (layers F.Cu B.Cu) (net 1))
 (via (at 144.78 97.79) (size 0.508) (drill 0.254) (layers F.Cu B.Cu) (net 1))
 (via (at 144.78 99.06) (size 0.508) (drill 0.254) (layers F.Cu B.Cu) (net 1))
 (segment (start 134.62 86.995) (end 134.62 92.56) (width 1.27) (layer F.Cu) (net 5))
 (segment (start 138.453 93.957) (end 138.453 93.98) (width 1.016) (layer F.Cu) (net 4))
 (segment (start 143.51 88.9) (end 138.453 93.957) (width 1.016) (layer F.Cu) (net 4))
 (segment (start 130.787 93.957) (end 130.787 93.98) (width 1.016) (layer F.Cu) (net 2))
 (segment (start 125.73 88.9) (end 130.787 93.957) (width 1.016) (layer F.Cu) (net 2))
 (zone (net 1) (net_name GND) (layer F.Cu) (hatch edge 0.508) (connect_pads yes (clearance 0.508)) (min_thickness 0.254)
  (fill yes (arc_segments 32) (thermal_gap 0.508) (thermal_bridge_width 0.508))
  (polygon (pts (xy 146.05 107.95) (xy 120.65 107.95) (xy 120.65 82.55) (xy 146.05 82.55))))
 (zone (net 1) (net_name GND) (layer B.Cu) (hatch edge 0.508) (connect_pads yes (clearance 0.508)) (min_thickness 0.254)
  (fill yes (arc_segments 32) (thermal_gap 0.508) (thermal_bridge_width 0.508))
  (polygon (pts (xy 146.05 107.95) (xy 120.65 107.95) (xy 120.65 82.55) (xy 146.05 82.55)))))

